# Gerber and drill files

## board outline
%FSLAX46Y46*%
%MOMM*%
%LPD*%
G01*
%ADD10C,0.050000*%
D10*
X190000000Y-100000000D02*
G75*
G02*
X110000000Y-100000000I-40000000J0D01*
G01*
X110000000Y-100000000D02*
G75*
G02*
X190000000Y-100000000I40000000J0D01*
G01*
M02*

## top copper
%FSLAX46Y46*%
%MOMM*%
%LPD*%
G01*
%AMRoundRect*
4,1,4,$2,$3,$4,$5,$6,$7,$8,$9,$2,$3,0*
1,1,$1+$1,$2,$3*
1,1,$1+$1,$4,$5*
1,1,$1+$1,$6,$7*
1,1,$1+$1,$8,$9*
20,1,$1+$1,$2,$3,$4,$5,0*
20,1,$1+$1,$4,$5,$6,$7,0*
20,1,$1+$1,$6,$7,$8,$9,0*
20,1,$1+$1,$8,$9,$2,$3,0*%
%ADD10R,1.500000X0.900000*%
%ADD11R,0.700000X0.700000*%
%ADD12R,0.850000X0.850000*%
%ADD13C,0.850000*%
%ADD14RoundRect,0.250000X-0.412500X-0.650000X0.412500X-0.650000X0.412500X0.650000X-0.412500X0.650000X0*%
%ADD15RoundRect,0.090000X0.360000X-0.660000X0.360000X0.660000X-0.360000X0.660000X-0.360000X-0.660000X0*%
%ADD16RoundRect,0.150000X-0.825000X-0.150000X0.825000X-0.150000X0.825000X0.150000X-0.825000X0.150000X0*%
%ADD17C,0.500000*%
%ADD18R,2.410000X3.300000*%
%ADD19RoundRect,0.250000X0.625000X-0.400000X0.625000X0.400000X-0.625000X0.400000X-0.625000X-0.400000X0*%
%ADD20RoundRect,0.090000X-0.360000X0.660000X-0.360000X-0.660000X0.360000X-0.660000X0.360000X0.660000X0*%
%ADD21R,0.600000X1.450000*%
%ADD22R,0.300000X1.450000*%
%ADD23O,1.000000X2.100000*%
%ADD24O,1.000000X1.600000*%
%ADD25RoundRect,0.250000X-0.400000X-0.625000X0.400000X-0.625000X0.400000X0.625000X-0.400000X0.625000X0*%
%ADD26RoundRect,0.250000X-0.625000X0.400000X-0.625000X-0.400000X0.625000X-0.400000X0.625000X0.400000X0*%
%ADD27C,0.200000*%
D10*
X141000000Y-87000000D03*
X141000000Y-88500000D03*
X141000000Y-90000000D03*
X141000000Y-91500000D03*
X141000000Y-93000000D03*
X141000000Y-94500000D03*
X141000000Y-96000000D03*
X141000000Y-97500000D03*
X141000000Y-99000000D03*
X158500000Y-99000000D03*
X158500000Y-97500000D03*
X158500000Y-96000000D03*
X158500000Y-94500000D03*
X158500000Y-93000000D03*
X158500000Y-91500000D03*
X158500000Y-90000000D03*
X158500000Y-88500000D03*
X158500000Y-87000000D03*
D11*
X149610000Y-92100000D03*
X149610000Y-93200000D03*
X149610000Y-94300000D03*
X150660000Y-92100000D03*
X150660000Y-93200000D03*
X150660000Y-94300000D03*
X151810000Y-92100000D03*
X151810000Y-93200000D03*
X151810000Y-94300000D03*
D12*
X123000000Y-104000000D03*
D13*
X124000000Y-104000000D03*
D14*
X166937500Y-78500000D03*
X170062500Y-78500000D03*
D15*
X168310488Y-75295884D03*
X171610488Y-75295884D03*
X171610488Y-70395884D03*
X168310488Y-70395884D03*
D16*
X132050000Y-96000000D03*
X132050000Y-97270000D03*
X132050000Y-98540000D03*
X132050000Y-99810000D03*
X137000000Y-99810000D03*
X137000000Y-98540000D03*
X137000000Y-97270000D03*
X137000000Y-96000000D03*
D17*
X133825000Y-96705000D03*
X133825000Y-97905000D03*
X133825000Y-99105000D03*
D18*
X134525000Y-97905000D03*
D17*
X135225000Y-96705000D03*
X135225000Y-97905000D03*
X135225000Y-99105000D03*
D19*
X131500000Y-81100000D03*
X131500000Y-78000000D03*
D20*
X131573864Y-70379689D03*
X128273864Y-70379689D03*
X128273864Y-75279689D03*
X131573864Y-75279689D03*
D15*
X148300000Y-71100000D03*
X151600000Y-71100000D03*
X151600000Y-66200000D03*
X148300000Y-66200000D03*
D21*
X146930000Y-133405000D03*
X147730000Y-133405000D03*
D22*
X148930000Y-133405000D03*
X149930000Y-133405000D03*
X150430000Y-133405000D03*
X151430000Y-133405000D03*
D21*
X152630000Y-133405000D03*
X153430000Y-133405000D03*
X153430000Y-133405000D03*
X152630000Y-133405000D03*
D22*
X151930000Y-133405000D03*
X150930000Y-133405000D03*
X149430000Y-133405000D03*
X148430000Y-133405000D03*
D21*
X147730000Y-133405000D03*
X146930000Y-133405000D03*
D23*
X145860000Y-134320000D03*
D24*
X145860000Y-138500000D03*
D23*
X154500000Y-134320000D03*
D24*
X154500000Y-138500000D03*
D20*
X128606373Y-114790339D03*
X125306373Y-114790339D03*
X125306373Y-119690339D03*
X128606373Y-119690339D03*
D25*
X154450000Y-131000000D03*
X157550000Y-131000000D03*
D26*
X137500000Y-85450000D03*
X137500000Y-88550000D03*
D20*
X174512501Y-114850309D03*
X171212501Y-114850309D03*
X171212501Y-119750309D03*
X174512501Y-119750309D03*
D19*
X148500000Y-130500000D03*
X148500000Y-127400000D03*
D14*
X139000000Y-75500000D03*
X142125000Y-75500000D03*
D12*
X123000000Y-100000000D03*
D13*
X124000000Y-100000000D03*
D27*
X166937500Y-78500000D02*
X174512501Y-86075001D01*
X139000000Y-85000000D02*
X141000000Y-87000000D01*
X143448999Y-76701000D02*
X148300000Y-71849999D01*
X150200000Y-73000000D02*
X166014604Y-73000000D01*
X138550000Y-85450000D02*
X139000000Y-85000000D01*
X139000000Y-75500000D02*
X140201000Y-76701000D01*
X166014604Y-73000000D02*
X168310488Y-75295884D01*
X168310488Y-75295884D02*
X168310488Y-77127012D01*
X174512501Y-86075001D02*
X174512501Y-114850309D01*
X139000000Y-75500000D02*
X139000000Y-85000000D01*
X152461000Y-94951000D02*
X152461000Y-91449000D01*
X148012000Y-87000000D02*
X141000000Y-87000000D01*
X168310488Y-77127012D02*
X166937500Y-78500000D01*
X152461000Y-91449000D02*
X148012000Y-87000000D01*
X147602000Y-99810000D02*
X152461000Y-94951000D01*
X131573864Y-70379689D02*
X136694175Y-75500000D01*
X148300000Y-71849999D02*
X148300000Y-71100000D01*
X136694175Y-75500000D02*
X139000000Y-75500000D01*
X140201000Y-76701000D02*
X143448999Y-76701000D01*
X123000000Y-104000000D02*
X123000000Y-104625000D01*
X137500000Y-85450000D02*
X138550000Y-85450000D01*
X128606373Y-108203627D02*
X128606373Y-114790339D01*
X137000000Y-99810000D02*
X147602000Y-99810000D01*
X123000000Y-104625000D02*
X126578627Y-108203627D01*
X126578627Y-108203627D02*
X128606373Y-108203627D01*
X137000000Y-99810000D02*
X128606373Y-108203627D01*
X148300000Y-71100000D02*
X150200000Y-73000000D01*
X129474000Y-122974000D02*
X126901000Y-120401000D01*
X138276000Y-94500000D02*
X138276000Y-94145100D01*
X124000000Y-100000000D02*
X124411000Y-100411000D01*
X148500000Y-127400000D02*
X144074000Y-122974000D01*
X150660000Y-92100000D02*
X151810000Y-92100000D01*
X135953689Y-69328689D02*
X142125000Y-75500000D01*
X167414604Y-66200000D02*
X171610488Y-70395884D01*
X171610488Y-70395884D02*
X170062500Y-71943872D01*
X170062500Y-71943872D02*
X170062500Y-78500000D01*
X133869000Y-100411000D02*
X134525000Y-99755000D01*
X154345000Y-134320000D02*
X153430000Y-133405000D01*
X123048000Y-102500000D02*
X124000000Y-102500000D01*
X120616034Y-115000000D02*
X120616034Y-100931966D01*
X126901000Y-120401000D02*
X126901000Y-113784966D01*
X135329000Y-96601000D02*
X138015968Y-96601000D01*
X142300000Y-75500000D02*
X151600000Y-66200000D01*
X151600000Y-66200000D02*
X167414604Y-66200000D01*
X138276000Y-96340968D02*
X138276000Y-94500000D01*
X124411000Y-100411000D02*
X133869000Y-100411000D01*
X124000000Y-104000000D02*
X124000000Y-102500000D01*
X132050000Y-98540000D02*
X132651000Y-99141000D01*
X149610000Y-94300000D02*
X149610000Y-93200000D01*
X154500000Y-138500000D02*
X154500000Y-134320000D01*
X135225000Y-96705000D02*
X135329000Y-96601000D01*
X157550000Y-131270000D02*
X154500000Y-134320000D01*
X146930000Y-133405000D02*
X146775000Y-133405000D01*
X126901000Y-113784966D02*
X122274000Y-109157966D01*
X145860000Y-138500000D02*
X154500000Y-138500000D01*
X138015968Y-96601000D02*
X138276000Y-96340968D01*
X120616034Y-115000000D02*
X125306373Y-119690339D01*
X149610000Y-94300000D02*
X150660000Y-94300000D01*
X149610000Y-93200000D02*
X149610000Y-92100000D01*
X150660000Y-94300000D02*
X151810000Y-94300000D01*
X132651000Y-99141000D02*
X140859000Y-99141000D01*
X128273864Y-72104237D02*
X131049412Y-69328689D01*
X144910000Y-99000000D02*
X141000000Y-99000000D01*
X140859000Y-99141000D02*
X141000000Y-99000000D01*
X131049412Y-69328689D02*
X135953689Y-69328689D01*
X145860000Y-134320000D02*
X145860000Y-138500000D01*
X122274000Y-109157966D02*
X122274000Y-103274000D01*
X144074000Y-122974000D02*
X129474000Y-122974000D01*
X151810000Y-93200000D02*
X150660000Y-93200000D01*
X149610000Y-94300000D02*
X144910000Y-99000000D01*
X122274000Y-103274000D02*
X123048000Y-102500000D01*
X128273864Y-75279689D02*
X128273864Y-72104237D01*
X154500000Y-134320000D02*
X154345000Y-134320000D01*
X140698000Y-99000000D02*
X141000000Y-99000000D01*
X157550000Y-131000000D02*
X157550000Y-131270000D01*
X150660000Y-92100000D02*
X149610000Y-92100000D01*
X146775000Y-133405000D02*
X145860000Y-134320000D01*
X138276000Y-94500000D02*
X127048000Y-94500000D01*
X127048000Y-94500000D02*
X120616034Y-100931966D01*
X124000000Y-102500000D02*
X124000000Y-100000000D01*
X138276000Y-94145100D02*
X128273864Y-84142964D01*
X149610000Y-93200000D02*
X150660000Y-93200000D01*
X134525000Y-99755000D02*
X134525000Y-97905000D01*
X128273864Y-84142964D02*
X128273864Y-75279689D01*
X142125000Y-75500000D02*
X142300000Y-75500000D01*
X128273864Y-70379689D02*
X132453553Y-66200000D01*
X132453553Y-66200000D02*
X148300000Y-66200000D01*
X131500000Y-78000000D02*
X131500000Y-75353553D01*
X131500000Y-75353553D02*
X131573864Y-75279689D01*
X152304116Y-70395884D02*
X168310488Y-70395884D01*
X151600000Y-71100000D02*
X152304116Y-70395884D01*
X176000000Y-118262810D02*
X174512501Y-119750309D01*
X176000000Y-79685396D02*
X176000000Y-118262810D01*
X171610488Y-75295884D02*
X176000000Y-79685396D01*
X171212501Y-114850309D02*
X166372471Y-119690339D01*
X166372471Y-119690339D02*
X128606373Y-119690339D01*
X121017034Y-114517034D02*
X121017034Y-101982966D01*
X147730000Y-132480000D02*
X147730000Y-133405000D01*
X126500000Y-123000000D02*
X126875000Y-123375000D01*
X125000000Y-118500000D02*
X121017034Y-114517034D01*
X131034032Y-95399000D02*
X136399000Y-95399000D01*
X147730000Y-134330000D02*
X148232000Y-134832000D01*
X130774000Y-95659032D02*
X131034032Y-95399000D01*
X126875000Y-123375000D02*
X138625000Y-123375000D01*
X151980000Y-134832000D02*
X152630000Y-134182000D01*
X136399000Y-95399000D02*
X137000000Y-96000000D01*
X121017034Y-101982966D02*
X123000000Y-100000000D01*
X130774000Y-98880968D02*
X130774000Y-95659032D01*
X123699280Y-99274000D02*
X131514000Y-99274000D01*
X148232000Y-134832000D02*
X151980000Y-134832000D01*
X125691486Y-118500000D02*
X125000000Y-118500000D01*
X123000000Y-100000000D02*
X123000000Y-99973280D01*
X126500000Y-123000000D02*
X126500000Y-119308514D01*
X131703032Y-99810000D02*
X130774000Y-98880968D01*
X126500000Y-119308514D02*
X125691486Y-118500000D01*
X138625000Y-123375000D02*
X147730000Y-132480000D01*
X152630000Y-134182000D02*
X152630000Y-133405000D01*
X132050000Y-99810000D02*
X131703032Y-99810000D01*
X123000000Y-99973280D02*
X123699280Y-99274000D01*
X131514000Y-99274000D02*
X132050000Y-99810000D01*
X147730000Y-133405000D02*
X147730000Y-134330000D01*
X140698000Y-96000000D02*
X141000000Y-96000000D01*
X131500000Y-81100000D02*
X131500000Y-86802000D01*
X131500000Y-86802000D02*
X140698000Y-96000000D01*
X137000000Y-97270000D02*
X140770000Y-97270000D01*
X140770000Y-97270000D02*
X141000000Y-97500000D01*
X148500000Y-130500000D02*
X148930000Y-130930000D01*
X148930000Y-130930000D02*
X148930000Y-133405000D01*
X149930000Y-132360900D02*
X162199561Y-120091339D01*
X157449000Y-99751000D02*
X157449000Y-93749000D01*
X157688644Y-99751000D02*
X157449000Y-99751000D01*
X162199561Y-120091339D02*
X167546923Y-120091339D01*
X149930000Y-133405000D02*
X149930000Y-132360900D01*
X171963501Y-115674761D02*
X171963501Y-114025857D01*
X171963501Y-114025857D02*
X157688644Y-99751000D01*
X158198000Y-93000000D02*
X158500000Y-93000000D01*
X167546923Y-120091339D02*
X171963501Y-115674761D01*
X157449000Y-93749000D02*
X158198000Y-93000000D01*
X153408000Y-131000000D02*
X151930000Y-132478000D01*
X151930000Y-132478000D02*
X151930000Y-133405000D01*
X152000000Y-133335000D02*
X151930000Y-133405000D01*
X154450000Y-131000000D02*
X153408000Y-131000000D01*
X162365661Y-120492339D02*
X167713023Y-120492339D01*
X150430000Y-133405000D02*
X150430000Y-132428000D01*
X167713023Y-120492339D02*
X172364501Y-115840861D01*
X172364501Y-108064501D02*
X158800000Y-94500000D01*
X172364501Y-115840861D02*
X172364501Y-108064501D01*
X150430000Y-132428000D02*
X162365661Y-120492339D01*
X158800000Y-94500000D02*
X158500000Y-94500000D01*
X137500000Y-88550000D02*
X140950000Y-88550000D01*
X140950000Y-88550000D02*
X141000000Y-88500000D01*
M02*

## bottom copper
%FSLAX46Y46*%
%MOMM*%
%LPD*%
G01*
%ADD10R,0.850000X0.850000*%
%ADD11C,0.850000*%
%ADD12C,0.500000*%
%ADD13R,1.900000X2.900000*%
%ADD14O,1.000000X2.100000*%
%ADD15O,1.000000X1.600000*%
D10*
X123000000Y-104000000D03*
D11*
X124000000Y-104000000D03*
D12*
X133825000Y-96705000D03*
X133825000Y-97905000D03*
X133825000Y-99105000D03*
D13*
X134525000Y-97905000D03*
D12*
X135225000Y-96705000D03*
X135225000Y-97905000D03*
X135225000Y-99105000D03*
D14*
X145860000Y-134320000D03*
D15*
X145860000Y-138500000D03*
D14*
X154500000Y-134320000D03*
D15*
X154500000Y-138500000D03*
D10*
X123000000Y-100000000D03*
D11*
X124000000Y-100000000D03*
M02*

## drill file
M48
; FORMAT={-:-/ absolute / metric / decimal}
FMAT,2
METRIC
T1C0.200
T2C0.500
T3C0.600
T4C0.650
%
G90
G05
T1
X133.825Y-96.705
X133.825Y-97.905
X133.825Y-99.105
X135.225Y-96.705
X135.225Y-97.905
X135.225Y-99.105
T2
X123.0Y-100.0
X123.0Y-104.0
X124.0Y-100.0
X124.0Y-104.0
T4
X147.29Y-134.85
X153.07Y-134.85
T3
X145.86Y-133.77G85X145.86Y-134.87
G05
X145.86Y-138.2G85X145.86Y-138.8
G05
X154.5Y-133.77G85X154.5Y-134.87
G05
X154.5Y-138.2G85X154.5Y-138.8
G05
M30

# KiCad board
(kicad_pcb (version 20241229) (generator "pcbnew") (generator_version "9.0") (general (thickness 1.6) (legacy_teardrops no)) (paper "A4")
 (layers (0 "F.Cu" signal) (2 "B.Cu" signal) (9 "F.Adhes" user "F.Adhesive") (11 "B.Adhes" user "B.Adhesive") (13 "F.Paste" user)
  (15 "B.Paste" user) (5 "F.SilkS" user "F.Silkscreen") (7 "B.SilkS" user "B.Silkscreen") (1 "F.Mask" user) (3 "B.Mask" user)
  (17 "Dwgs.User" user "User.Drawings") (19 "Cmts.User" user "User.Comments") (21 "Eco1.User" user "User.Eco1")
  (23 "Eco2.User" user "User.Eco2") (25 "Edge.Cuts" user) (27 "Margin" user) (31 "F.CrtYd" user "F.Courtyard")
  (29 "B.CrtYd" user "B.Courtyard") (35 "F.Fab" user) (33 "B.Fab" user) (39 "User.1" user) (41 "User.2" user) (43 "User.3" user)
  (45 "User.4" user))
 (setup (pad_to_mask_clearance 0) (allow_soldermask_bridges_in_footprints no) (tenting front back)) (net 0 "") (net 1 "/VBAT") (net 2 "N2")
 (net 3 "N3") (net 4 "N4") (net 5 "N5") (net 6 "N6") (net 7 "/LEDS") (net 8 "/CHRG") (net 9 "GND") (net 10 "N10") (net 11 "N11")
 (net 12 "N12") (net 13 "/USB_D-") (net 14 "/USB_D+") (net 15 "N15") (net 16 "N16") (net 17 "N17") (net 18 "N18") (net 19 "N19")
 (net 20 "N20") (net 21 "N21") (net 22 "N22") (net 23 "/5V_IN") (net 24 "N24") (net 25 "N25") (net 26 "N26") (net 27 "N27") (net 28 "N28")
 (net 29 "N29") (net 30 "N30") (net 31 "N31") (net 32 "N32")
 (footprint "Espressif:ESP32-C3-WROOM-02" (layer "F.Cu") (at 149.75 92.9)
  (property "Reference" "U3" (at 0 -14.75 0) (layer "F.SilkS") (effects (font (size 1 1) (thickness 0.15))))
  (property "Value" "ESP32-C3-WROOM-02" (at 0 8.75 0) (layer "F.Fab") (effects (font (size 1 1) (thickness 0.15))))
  (pad "1" smd rect (at -8.75 -5.9) (size 1.5 0.9) (layers "F.Cu" "F.Mask" "F.Paste") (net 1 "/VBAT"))
  (pad "2" smd rect (at -8.75 -4.4) (size 1.5 0.9) (layers "F.Cu" "F.Mask" "F.Paste") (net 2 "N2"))
  (pad "3" smd rect (at -8.75 -2.9) (size 1.5 0.9) (layers "F.Cu" "F.Mask" "F.Paste") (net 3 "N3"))
  (pad "4" smd rect (at -8.75 -1.4) (size 1.5 0.9) (layers "F.Cu" "F.Mask" "F.Paste") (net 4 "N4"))
  (pad "5" smd rect (at -8.75 0.1) (size 1.5 0.9) (layers "F.Cu" "F.Mask" "F.Paste") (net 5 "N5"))
  (pad "6" smd rect (at -8.75 1.6) (size 1.5 0.9) (layers "F.Cu" "F.Mask" "F.Paste") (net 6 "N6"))
  (pad "7" smd rect (at -8.75 3.1) (size 1.5 0.9) (layers "F.Cu" "F.Mask" "F.Paste") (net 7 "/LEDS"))
  (pad "8" smd rect (at -8.75 4.6) (size 1.5 0.9) (layers "F.Cu" "F.Mask" "F.Paste") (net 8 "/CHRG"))
  (pad "9" smd rect (at -8.75 6.1) (size 1.5 0.9) (layers "F.Cu" "F.Mask" "F.Paste") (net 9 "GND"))
  (pad "10" smd rect (at 8.75 6.1 180) (size 1.5 0.9) (layers "F.Cu" "F.Mask" "F.Paste") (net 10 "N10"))
  (pad "11" smd rect (at 8.75 4.6 180) (size 1.5 0.9) (layers "F.Cu" "F.Mask" "F.Paste") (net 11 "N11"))
  (pad "12" smd rect (at 8.75 3.1 180) (size 1.5 0.9) (layers "F.Cu" "F.Mask" "F.Paste") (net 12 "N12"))
  (pad "13" smd rect (at 8.75 1.6 180) (size 1.5 0.9) (layers "F.Cu" "F.Mask" "F.Paste") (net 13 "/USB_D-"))
  (pad "14" smd rect (at 8.75 0.1 180) (size 1.5 0.9) (layers "F.Cu" "F.Mask" "F.Paste") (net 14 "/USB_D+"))
  (pad "15" smd rect (at 8.75 -1.4 180) (size 1.5 0.9) (layers "F.Cu" "F.Mask" "F.Paste") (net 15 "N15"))
  (pad "16" smd rect (at 8.75 -2.9 180) (size 1.5 0.9) (layers "F.Cu" "F.Mask" "F.Paste") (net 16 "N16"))
  (pad "17" smd rect (at 8.75 -4.4 180) (size 1.5 0.9) (layers "F.Cu" "F.Mask" "F.Paste") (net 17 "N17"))
  (pad "18" smd rect (at 8.75 -5.9 180) (size 1.5 0.9) (layers "F.Cu" "F.Mask" "F.Paste") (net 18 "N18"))
  (pad "19" smd rect (at -0.14 -0.8 180) (size 0.7 0.7) (layers "F.Cu" "F.Mask" "F.Paste") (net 9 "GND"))
  (pad "19" smd rect (at -0.14 0.3 180) (size 0.7 0.7) (layers "F.Cu" "F.Mask" "F.Paste") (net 9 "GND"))
  (pad "19" smd rect (at -0.14 1.4 180) (size 0.7 0.7) (layers "F.Cu" "F.Mask" "F.Paste") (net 9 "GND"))
  (pad "19" smd rect (at 0.91 -0.8 180) (size 0.7 0.7) (layers "F.Cu" "F.Mask" "F.Paste") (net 9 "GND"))
  (pad "19" smd rect (at 0.91 0.3 180) (size 0.7 0.7) (layers "F.Cu" "F.Mask" "F.Paste") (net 9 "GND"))
  (pad "19" smd rect (at 0.91 1.4 180) (size 0.7 0.7) (layers "F.Cu" "F.Mask" "F.Paste") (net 9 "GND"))
  (pad "19" smd rect (at 2.06 -0.8 180) (size 0.7 0.7) (layers "F.Cu" "F.Mask" "F.Paste") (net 9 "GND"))
  (pad "19" smd rect (at 2.06 0.3 180) (size 0.7 0.7) (layers "F.Cu" "F.Mask" "F.Paste") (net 9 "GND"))
  (pad "19" smd rect (at 2.06 1.4 180) (size 0.7 0.7) (layers "F.Cu" "F.Mask" "F.Paste") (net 9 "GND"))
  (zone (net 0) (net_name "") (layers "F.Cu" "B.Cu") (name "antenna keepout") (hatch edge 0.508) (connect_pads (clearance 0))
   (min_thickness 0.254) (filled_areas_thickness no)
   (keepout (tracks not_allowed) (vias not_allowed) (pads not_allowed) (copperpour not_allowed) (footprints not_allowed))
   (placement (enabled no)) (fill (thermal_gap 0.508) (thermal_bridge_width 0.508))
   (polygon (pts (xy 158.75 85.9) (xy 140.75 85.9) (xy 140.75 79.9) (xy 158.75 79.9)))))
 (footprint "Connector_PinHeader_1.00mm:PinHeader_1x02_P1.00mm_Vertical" (layer "F.Cu") (at 123 104 90)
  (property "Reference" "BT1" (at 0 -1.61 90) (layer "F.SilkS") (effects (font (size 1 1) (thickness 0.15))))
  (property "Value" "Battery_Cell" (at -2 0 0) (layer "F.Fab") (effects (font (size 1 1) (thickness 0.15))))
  (pad "1" thru_hole rect (at 0 0 90) (size 0.85 0.85) (drill 0.5) (layers "*.Cu" "*.Mask") (remove_unused_layers no) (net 1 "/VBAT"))
  (pad "2" thru_hole circle (at 0 1 90) (size 0.85 0.85) (drill 0.5) (layers "*.Cu" "*.Mask") (remove_unused_layers no) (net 9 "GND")))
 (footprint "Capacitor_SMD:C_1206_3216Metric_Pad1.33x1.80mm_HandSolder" (layer "F.Cu") (at 168.5 78.5)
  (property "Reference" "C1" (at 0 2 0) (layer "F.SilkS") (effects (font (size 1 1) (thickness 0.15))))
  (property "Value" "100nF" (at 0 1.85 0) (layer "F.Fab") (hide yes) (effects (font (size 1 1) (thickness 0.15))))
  (pad "1" smd roundrect (at -1.5625 0) (size 1.325 1.8) (layers "F.Cu" "F.Mask" "F.Paste") (roundrect_rratio 0.188679) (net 1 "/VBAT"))
  (pad "2" smd roundrect (at 1.5625 0) (size 1.325 1.8) (layers "F.Cu" "F.Mask" "F.Paste") (roundrect_rratio 0.188679) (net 9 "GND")))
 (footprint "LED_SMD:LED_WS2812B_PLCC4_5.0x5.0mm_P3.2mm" (layer "F.Cu") (at 169.960488 72.845884 90)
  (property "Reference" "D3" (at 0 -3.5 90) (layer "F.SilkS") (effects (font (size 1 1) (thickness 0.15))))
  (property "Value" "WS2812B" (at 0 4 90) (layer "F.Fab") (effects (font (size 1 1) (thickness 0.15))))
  (pad "1" smd roundrect (at -2.45 -1.65 90) (size 1.5 0.9) (layers "F.Cu" "F.Mask" "F.Paste") (roundrect_rratio 0.1) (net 1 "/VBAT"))
  (pad "2" smd roundrect (at -2.45 1.65 90) (size 1.5 0.9) (layers "F.Cu" "F.Mask" "F.Paste") (roundrect_rratio 0.1) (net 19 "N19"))
  (pad "3" smd roundrect (at 2.45 1.65 90) (size 1.5 0.9) (layers "F.Cu" "F.Mask" "F.Paste") (roundrect_rratio 0.1) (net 9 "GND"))
  (pad "4" smd roundrect (at 2.45 -1.65 90) (size 1.5 0.9) (layers "F.Cu" "F.Mask" "F.Paste") (roundrect_rratio 0.1) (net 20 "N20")))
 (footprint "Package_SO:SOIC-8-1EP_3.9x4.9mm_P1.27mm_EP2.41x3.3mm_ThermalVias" (layer "F.Cu") (at 134.525 97.905)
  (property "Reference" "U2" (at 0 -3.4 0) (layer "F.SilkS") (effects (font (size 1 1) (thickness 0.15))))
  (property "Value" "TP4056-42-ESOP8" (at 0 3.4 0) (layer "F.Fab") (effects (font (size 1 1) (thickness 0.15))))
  (pad "" smd roundrect (at -0.6 -0.825) (size 1.01 1.38) (layers "F.Paste") (roundrect_rratio 0.247525))
  (pad "" smd roundrect (at -0.6 0.825) (size 1.01 1.38) (layers "F.Paste") (roundrect_rratio 0.247525))
  (pad "" smd roundrect (at 0.6 -0.825) (size 1.01 1.38) (layers "F.Paste") (roundrect_rratio 0.247525))
  (pad "" smd roundrect (at 0.6 0.825) (size 1.01 1.38) (layers "F.Paste") (roundrect_rratio 0.247525))
  (pad "1" smd roundrect (at -2.475 -1.905) (size 1.95 0.6) (layers "F.Cu" "F.Mask" "F.Paste") (roundrect_rratio 0.25) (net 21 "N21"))
  (pad "2" smd roundrect (at -2.475 -0.635) (size 1.95 0.6) (layers "F.Cu" "F.Mask" "F.Paste") (roundrect_rratio 0.25) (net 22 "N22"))
  (pad "3" smd roundrect (at -2.475 0.635) (size 1.95 0.6) (layers "F.Cu" "F.Mask" "F.Paste") (roundrect_rratio 0.25) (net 9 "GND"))
  (pad "4" smd roundrect (at -2.475 1.905) (size 1.95 0.6) (layers "F.Cu" "F.Mask" "F.Paste") (roundrect_rratio 0.25) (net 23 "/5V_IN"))
  (pad "5" smd roundrect (at 2.475 1.905) (size 1.95 0.6) (layers "F.Cu" "F.Mask" "F.Paste") (roundrect_rratio 0.25) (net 1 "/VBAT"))
  (pad "6" smd roundrect (at 2.475 0.635) (size 1.95 0.6) (layers "F.Cu" "F.Mask" "F.Paste") (roundrect_rratio 0.25) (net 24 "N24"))
  (pad "7" smd roundrect (at 2.475 -0.635) (size 1.95 0.6) (layers "F.Cu" "F.Mask" "F.Paste") (roundrect_rratio 0.25) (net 8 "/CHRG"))
  (pad "8" smd roundrect (at 2.475 -1.905) (size 1.95 0.6) (layers "F.Cu" "F.Mask" "F.Paste") (roundrect_rratio 0.25) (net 23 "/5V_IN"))
  (pad "9" thru_hole circle (at -0.7 -1.2) (size 0.5 0.5) (drill 0.2) (layers "*.Cu") (remove_unused_layers no) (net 9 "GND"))
  (pad "9" thru_hole circle (at -0.7 0) (size 0.5 0.5) (drill 0.2) (layers "*.Cu") (remove_unused_layers no) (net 9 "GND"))
  (pad "9" thru_hole circle (at -0.7 1.2) (size 0.5 0.5) (drill 0.2) (layers "*.Cu") (remove_unused_layers no) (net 9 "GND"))
  (pad "9" smd rect (at 0 0) (size 1.9 2.9) (layers "B.Cu") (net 9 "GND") (zone_connect 2))
  (pad "9" smd rect (at 0 0) (size 2.41 3.3) (layers "F.Cu" "F.Mask") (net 9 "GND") (zone_connect 2))
  (pad "9" thru_hole circle (at 0.7 -1.2) (size 0.5 0.5) (drill 0.2) (layers "*.Cu") (remove_unused_layers no) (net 9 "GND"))
  (pad "9" thru_hole circle (at 0.7 0) (size 0.5 0.5) (drill 0.2) (layers "*.Cu") (remove_unused_layers no) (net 9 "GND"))
  (pad "9" thru_hole circle (at 0.7 1.2) (size 0.5 0.5) (drill 0.2) (layers "*.Cu") (remove_unused_layers no) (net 9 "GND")))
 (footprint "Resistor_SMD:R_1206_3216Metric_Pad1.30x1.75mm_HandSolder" (layer "F.Cu") (at 131.5 79.55 90)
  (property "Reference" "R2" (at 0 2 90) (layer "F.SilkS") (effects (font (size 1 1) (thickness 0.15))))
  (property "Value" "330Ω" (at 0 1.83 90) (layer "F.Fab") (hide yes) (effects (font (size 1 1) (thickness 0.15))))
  (pad "1" smd roundrect (at -1.55 0 90) (size 1.3 1.75) (layers "F.Cu" "F.Mask" "F.Paste") (roundrect_rratio 0.192308) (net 7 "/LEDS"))
  (pad "2" smd roundrect (at 1.55 0 90) (size 1.3 1.75) (layers "F.Cu" "F.Mask" "F.Paste") (roundrect_rratio 0.192308) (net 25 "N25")))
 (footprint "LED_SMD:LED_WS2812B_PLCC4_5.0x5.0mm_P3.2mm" (layer "F.Cu") (at 129.923864 72.829689 -90)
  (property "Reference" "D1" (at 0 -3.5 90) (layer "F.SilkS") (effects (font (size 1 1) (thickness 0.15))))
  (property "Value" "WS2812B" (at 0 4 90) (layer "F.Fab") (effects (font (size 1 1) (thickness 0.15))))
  (pad "1" smd roundrect (at -2.45 -1.65 270) (size 1.5 0.9) (layers "F.Cu" "F.Mask" "F.Paste") (roundrect_rratio 0.1) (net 1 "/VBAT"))
  (pad "2" smd roundrect (at -2.45 1.65 270) (size 1.5 0.9) (layers "F.Cu" "F.Mask" "F.Paste") (roundrect_rratio 0.1) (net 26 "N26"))
  (pad "3" smd roundrect (at 2.45 1.65 270) (size 1.5 0.9) (layers "F.Cu" "F.Mask" "F.Paste") (roundrect_rratio 0.1) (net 9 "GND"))
  (pad "4" smd roundrect (at 2.45 -1.65 270) (size 1.5 0.9) (layers "F.Cu" "F.Mask" "F.Paste") (roundrect_rratio 0.1) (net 25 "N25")))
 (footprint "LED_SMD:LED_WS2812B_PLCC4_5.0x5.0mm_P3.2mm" (layer "F.Cu") (at 149.95 68.65 90)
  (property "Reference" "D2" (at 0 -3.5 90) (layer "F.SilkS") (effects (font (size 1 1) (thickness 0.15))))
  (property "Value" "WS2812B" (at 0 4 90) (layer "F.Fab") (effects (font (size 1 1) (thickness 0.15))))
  (pad "1" smd roundrect (at -2.45 -1.65 90) (size 1.5 0.9) (layers "F.Cu" "F.Mask" "F.Paste") (roundrect_rratio 0.1) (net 1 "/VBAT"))
  (pad "2" smd roundrect (at -2.45 1.65 90) (size 1.5 0.9) (layers "F.Cu" "F.Mask" "F.Paste") (roundrect_rratio 0.1) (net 20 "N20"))
  (pad "3" smd roundrect (at 2.45 1.65 90) (size 1.5 0.9) (layers "F.Cu" "F.Mask" "F.Paste") (roundrect_rratio 0.1) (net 9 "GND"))
  (pad "4" smd roundrect (at 2.45 -1.65 90) (size 1.5 0.9) (layers "F.Cu" "F.Mask" "F.Paste") (roundrect_rratio 0.1) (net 26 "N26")))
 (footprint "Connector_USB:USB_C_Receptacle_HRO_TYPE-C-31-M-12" (layer "F.Cu") (at 150.18 137.45)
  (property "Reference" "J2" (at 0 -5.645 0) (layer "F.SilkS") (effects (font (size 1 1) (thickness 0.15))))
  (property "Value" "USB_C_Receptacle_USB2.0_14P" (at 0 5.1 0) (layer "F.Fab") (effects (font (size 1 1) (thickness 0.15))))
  (pad "" np_thru_hole circle (at -2.89 -2.6) (size 0.65 0.65) (drill 0.65) (layers "*.Cu" "*.Mask"))
  (pad "" np_thru_hole circle (at 2.89 -2.6) (size 0.65 0.65) (drill 0.65) (layers "*.Cu" "*.Mask"))
  (pad "A1" smd rect (at -3.25 -4.045) (size 0.6 1.45) (layers "F.Cu" "F.Mask" "F.Paste") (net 9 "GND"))
  (pad "A4" smd rect (at -2.45 -4.045) (size 0.6 1.45) (layers "F.Cu" "F.Mask" "F.Paste") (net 23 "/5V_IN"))
  (pad "A5" smd rect (at -1.25 -4.045) (size 0.3 1.45) (layers "F.Cu" "F.Mask" "F.Paste") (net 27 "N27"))
  (pad "A6" smd rect (at -0.25 -4.045) (size 0.3 1.45) (layers "F.Cu" "F.Mask" "F.Paste") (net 14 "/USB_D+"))
  (pad "A7" smd rect (at 0.25 -4.045) (size 0.3 1.45) (layers "F.Cu" "F.Mask" "F.Paste") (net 13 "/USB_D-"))
  (pad "A8" smd rect (at 1.25 -4.045) (size 0.3 1.45) (layers "F.Cu" "F.Mask" "F.Paste"))
  (pad "A9" smd rect (at 2.45 -4.045) (size 0.6 1.45) (layers "F.Cu" "F.Mask" "F.Paste") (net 23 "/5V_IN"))
  (pad "A12" smd rect (at 3.25 -4.045) (size 0.6 1.45) (layers "F.Cu" "F.Mask" "F.Paste") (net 9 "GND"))
  (pad "B1" smd rect (at 3.25 -4.045) (size 0.6 1.45) (layers "F.Cu" "F.Mask" "F.Paste") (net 9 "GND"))
  (pad "B4" smd rect (at 2.45 -4.045) (size 0.6 1.45) (layers "F.Cu" "F.Mask" "F.Paste") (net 23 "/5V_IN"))
  (pad "B5" smd rect (at 1.75 -4.045) (size 0.3 1.45) (layers "F.Cu" "F.Mask" "F.Paste") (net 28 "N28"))
  (pad "B6" smd rect (at 0.75 -4.045) (size 0.3 1.45) (layers "F.Cu" "F.Mask" "F.Paste") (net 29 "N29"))
  (pad "B7" smd rect (at -0.75 -4.045) (size 0.3 1.45) (layers "F.Cu" "F.Mask" "F.Paste") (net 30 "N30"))
  (pad "B8" smd rect (at -1.75 -4.045) (size 0.3 1.45) (layers "F.Cu" "F.Mask" "F.Paste"))
  (pad "B9" smd rect (at -2.45 -4.045) (size 0.6 1.45) (layers "F.Cu" "F.Mask" "F.Paste") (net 23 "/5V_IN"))
  (pad "B12" smd rect (at -3.25 -4.045) (size 0.6 1.45) (layers "F.Cu" "F.Mask" "F.Paste") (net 9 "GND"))
  (pad "S1" thru_hole oval (at -4.32 -3.13) (size 1 2.1) (drill oval 0.6 1.7) (layers "*.Cu" "*.Mask") (remove_unused_layers no)
   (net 9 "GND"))
  (pad "S1" thru_hole oval (at -4.32 1.05) (size 1 1.6) (drill oval 0.6 1.2) (layers "*.Cu" "*.Mask") (remove_unused_layers no)
   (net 9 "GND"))
  (pad "S1" thru_hole oval (at 4.32 -3.13) (size 1 2.1) (drill oval 0.6 1.7) (layers "*.Cu" "*.Mask") (remove_unused_layers no)
   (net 9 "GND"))
  (pad "S1" thru_hole oval (at 4.32 1.05) (size 1 1.6) (drill oval 0.6 1.2) (layers "*.Cu" "*.Mask") (remove_unused_layers no) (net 9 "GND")))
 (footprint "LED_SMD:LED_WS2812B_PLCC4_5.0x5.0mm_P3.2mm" (layer "F.Cu") (at 126.956373 117.240339 -90)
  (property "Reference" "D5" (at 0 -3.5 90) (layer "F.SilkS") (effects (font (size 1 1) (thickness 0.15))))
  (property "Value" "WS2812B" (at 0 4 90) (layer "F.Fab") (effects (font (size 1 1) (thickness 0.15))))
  (pad "1" smd roundrect (at -2.45 -1.65 270) (size 1.5 0.9) (layers "F.Cu" "F.Mask" "F.Paste") (roundrect_rratio 0.1) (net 1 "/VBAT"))
  (pad "2" smd roundrect (at -2.45 1.65 270) (size 1.5 0.9) (layers "F.Cu" "F.Mask" "F.Paste") (roundrect_rratio 0.1) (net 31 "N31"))
  (pad "3" smd roundrect (at 2.45 1.65 270) (size 1.5 0.9) (layers "F.Cu" "F.Mask" "F.Paste") (roundrect_rratio 0.1) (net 9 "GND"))
  (pad "4" smd roundrect (at 2.45 -1.65 270) (size 1.5 0.9) (layers "F.Cu" "F.Mask" "F.Paste") (roundrect_rratio 0.1) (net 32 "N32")))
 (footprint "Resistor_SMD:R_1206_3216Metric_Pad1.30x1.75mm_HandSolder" (layer "F.Cu") (at 156 131)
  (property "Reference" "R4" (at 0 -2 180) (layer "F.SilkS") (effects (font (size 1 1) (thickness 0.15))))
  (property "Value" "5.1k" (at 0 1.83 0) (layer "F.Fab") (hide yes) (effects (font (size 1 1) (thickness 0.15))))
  (pad "1" smd roundrect (at -1.55 0) (size 1.3 1.75) (layers "F.Cu" "F.Mask" "F.Paste") (roundrect_rratio 0.192308) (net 28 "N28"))
  (pad "2" smd roundrect (at 1.55 0) (size 1.3 1.75) (layers "F.Cu" "F.Mask" "F.Paste") (roundrect_rratio 0.192308) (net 9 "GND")))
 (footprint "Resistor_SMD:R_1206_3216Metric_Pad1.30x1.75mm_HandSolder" (layer "F.Cu") (at 137.5 87 -90)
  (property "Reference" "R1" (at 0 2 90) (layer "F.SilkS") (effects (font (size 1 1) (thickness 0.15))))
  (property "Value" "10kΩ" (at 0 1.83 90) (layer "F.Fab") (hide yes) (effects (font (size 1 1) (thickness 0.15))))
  (pad "1" smd roundrect (at -1.55 0 270) (size 1.3 1.75) (layers "F.Cu" "F.Mask" "F.Paste") (roundrect_rratio 0.192308) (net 1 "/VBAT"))
  (pad "2" smd roundrect (at 1.55 0 270) (size 1.3 1.75) (layers "F.Cu" "F.Mask" "F.Paste") (roundrect_rratio 0.192308) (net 2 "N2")))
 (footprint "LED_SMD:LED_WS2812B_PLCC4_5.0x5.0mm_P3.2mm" (layer "F.Cu") (at 172.862501 117.300309 -90)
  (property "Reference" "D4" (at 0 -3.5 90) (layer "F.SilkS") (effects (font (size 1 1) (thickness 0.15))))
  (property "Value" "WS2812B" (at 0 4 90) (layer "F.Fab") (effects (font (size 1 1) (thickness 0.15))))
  (pad "1" smd roundrect (at -2.45 -1.65 270) (size 1.5 0.9) (layers "F.Cu" "F.Mask" "F.Paste") (roundrect_rratio 0.1) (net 1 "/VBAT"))
  (pad "2" smd roundrect (at -2.45 1.65 270) (size 1.5 0.9) (layers "F.Cu" "F.Mask" "F.Paste") (roundrect_rratio 0.1) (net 32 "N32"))
  (pad "3" smd roundrect (at 2.45 1.65 270) (size 1.5 0.9) (layers "F.Cu" "F.Mask" "F.Paste") (roundrect_rratio 0.1) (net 9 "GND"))
  (pad "4" smd roundrect (at 2.45 -1.65 270) (size 1.5 0.9) (layers "F.Cu" "F.Mask" "F.Paste") (roundrect_rratio 0.1) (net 19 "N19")))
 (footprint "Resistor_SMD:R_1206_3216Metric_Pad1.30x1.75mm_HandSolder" (layer "F.Cu") (at 148.5 128.95 90)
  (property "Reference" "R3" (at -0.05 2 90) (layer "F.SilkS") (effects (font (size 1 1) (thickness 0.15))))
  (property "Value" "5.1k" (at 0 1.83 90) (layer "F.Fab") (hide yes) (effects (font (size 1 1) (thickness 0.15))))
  (pad "1" smd roundrect (at -1.55 0 90) (size 1.3 1.75) (layers "F.Cu" "F.Mask" "F.Paste") (roundrect_rratio 0.192308) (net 27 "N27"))
  (pad "2" smd roundrect (at 1.55 0 90) (size 1.3 1.75) (layers "F.Cu" "F.Mask" "F.Paste") (roundrect_rratio 0.192308) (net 9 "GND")))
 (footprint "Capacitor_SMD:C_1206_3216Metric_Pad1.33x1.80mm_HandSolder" (layer "F.Cu") (at 140.5625 75.5)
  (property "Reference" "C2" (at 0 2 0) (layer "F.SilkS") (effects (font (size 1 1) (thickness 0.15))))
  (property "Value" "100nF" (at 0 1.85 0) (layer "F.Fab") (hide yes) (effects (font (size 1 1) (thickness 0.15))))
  (pad "1" smd roundrect (at -1.5625 0) (size 1.325 1.8) (layers "F.Cu" "F.Mask" "F.Paste") (roundrect_rratio 0.188679) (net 1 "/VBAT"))
  (pad "2" smd roundrect (at 1.5625 0) (size 1.325 1.8) (layers "F.Cu" "F.Mask" "F.Paste") (roundrect_rratio 0.188679) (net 9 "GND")))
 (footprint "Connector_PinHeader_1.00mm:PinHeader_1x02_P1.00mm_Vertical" (layer "F.Cu") (at 123 100 90)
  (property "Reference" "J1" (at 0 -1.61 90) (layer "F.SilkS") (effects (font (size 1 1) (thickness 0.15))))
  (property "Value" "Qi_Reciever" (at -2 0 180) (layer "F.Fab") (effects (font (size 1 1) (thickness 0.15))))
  (pad "1" thru_hole rect (at 0 0 90) (size 0.85 0.85) (drill 0.5) (layers "*.Cu" "*.Mask") (remove_unused_layers no) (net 23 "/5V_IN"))
  (pad "2" thru_hole circle (at 0 1 90) (size 0.85 0.85) (drill 0.5) (layers "*.Cu" "*.Mask") (remove_unused_layers no) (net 9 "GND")))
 (gr_circle (center 150 100) (end 190 100) (stroke (width 0.05) (type default)) (fill no) (layer "Edge.Cuts"))
 (segment (start 166.9375 78.5) (end 174.512501 86.075001) (width 0.2) (layer "F.Cu") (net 1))
 (segment (start 139 85) (end 141 87) (width 0.2) (layer "F.Cu") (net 1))
 (segment (start 143.448999 76.701) (end 148.3 71.849999) (width 0.2) (layer "F.Cu") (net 1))
 (segment (start 150.2 73) (end 166.014604 73) (width 0.2) (layer "F.Cu") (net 1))
 (segment (start 138.55 85.45) (end 139 85) (width 0.2) (layer "F.Cu") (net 1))
 (segment (start 139 75.5) (end 140.201 76.701) (width 0.2) (layer "F.Cu") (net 1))
 (segment (start 166.014604 73) (end 168.310488 75.295884) (width 0.2) (layer "F.Cu") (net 1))
 (segment (start 168.310488 75.295884) (end 168.310488 77.127012) (width 0.2) (layer "F.Cu") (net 1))
 (segment (start 174.512501 86.075001) (end 174.512501 114.850309) (width 0.2) (layer "F.Cu") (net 1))
 (segment (start 139 75.5) (end 139 85) (width 0.2) (layer "F.Cu") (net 1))
 (segment (start 152.461 94.951) (end 152.461 91.449) (width 0.2) (layer "F.Cu") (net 1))
 (segment (start 148.012 87) (end 141 87) (width 0.2) (layer "F.Cu") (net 1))
 (segment (start 168.310488 77.127012) (end 166.9375 78.5) (width 0.2) (layer "F.Cu") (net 1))
 (segment (start 152.461 91.449) (end 148.012 87) (width 0.2) (layer "F.Cu") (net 1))
 (segment (start 147.602 99.81) (end 152.461 94.951) (width 0.2) (layer "F.Cu") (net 1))
 (segment (start 131.573864 70.379689) (end 136.694175 75.5) (width 0.2) (layer "F.Cu") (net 1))
 (segment (start 148.3 71.849999) (end 148.3 71.1) (width 0.2) (layer "F.Cu") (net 1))
 (segment (start 136.694175 75.5) (end 139 75.5) (width 0.2) (layer "F.Cu") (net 1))
 (segment (start 140.201 76.701) (end 143.448999 76.701) (width 0.2) (layer "F.Cu") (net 1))
 (segment (start 123 104) (end 123 104.625) (width 0.2) (layer "F.Cu") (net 1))
 (segment (start 137.5 85.45) (end 138.55 85.45) (width 0.2) (layer "F.Cu") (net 1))
 (segment (start 128.606373 108.203627) (end 128.606373 114.790339) (width 0.2) (layer "F.Cu") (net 1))
 (segment (start 137 99.81) (end 147.602 99.81) (width 0.2) (layer "F.Cu") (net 1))
 (segment (start 123 104.625) (end 126.578627 108.203627) (width 0.2) (layer "F.Cu") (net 1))
 (segment (start 126.578627 108.203627) (end 128.606373 108.203627) (width 0.2) (layer "F.Cu") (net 1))
 (segment (start 137 99.81) (end 128.606373 108.203627) (width 0.2) (layer "F.Cu") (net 1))
 (segment (start 148.3 71.1) (end 150.2 73) (width 0.2) (layer "F.Cu") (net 1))
 (segment (start 129.474 122.974) (end 126.901 120.401) (width 0.2) (layer "F.Cu") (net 9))
 (segment (start 138.276 94.5) (end 138.276 94.1451) (width 0.2) (layer "F.Cu") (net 9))
 (segment (start 124 100) (end 124.411 100.411) (width 0.2) (layer "F.Cu") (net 9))
 (segment (start 148.5 127.4) (end 144.074 122.974) (width 0.2) (layer "F.Cu") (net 9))
 (segment (start 150.66 92.1) (end 151.81 92.1) (width 0.2) (layer "F.Cu") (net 9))
 (segment (start 135.953689 69.328689) (end 142.125 75.5) (width 0.2) (layer "F.Cu") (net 9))
 (segment (start 167.414604 66.2) (end 171.610488 70.395884) (width 0.2) (layer "F.Cu") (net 9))
 (segment (start 171.610488 70.395884) (end 170.0625 71.943872) (width 0.2) (layer "F.Cu") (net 9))
 (segment (start 170.0625 71.943872) (end 170.0625 78.5) (width 0.2) (layer "F.Cu") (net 9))
 (segment (start 133.869 100.411) (end 134.525 99.755) (width 0.2) (layer "F.Cu") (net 9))
 (segment (start 154.345 134.32) (end 153.43 133.405) (width 0.2) (layer "F.Cu") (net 9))
 (segment (start 123.048 102.5) (end 124 102.5) (width 0.2) (layer "F.Cu") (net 9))
 (segment (start 120.616034 115) (end 120.616034 100.931966) (width 0.2) (layer "F.Cu") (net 9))
 (segment (start 126.901 120.401) (end 126.901 113.784966) (width 0.2) (layer "F.Cu") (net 9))
 (segment (start 135.329 96.601) (end 138.015968 96.601) (width 0.2) (layer "F.Cu") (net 9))
 (segment (start 142.3 75.5) (end 151.6 66.2) (width 0.2) (layer "F.Cu") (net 9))
 (segment (start 151.6 66.2) (end 167.414604 66.2) (width 0.2) (layer "F.Cu") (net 9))
 (segment (start 138.276 96.340968) (end 138.276 94.5) (width 0.2) (layer "F.Cu") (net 9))
 (segment (start 124.411 100.411) (end 133.869 100.411) (width 0.2) (layer "F.Cu") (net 9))
 (segment (start 124 104) (end 124 102.5) (width 0.2) (layer "F.Cu") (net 9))
 (segment (start 132.05 98.54) (end 132.651 99.141) (width 0.2) (layer "F.Cu") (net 9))
 (segment (start 149.61 94.3) (end 149.61 93.2) (width 0.2) (layer "F.Cu") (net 9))
 (segment (start 154.5 138.5) (end 154.5 134.32) (width 0.2) (layer "F.Cu") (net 9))
 (segment (start 135.225 96.705) (end 135.329 96.601) (width 0.2) (layer "F.Cu") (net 9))
 (segment (start 157.55 131.27) (end 154.5 134.32) (width 0.2) (layer "F.Cu") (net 9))
 (segment (start 146.93 133.405) (end 146.775 133.405) (width 0.2) (layer "F.Cu") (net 9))
 (segment (start 126.901 113.784966) (end 122.274 109.157966) (width 0.2) (layer "F.Cu") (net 9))
 (segment (start 145.86 138.5) (end 154.5 138.5) (width 0.2) (layer "F.Cu") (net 9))
 (segment (start 138.015968 96.601) (end 138.276 96.340968) (width 0.2) (layer "F.Cu") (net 9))
 (segment (start 120.616034 115) (end 125.306373 119.690339) (width 0.2) (layer "F.Cu") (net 9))
 (segment (start 149.61 94.3) (end 150.66 94.3) (width 0.2) (layer "F.Cu") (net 9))
 (segment (start 149.61 93.2) (end 149.61 92.1) (width 0.2) (layer "F.Cu") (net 9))
 (segment (start 150.66 94.3) (end 151.81 94.3) (width 0.2) (layer "F.Cu") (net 9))
 (segment (start 132.651 99.141) (end 140.859 99.141) (width 0.2) (layer "F.Cu") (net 9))
 (segment (start 128.273864 72.104237) (end 131.049412 69.328689) (width 0.2) (layer "F.Cu") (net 9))
 (segment (start 144.91 99) (end 141 99) (width 0.2) (layer "F.Cu") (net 9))
 (segment (start 140.859 99.141) (end 141 99) (width 0.2) (layer "F.Cu") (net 9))
 (segment (start 131.049412 69.328689) (end 135.953689 69.328689) (width 0.2) (layer "F.Cu") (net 9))
 (segment (start 145.86 134.32) (end 145.86 138.5) (width 0.2) (layer "F.Cu") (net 9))
 (segment (start 122.274 109.157966) (end 122.274 103.274) (width 0.2) (layer "F.Cu") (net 9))
 (segment (start 144.074 122.974) (end 129.474 122.974) (width 0.2) (layer "F.Cu") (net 9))
 (segment (start 151.81 93.2) (end 150.66 93.2) (width 0.2) (layer "F.Cu") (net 9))
 (segment (start 149.61 94.3) (end 144.91 99) (width 0.2) (layer "F.Cu") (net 9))
 (segment (start 122.274 103.274) (end 123.048 102.5) (width 0.2) (layer "F.Cu") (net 9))
 (segment (start 128.273864 75.279689) (end 128.273864 72.104237) (width 0.2) (layer "F.Cu") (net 9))
 (segment (start 154.5 134.32) (end 154.345 134.32) (width 0.2) (layer "F.Cu") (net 9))
 (segment (start 140.698 99) (end 141 99) (width 0.2) (layer "F.Cu") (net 9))
 (segment (start 157.55 131) (end 157.55 131.27) (width 0.2) (layer "F.Cu") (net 9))
 (segment (start 150.66 92.1) (end 149.61 92.1) (width 0.2) (layer "F.Cu") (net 9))
 (segment (start 146.775 133.405) (end 145.86 134.32) (width 0.2) (layer "F.Cu") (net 9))
 (segment (start 138.276 94.5) (end 127.048 94.5) (width 0.2) (layer "F.Cu") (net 9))
 (segment (start 127.048 94.5) (end 120.616034 100.931966) (width 0.2) (layer "F.Cu") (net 9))
 (segment (start 124 102.5) (end 124 100) (width 0.2) (layer "F.Cu") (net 9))
 (segment (start 138.276 94.1451) (end 128.273864 84.142964) (width 0.2) (layer "F.Cu") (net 9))
 (segment (start 149.61 93.2) (end 150.66 93.2) (width 0.2) (layer "F.Cu") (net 9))
 (segment (start 134.525 99.755) (end 134.525 97.905) (width 0.2) (layer "F.Cu") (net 9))
 (segment (start 128.273864 84.142964) (end 128.273864 75.279689) (width 0.2) (layer "F.Cu") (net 9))
 (segment (start 142.125 75.5) (end 142.3 75.5) (width 0.2) (layer "F.Cu") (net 9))
 (segment (start 128.273864 70.379689) (end 132.453553 66.2) (width 0.2) (layer "F.Cu") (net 26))
 (segment (start 132.453553 66.2) (end 148.3 66.2) (width 0.2) (layer "F.Cu") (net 26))
 (segment (start 131.5 78) (end 131.5 75.353553) (width 0.2) (layer "F.Cu") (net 25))
 (segment (start 131.5 75.353553) (end 131.573864 75.279689) (width 0.2) (layer "F.Cu") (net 25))
 (segment (start 152.304116 70.395884) (end 168.310488 70.395884) (width 0.2) (layer "F.Cu") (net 20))
 (segment (start 151.6 71.1) (end 152.304116 70.395884) (width 0.2) (layer "F.Cu") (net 20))
 (segment (start 176 118.26281) (end 174.512501 119.750309) (width 0.2) (layer "F.Cu") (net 19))
 (segment (start 176 79.685396) (end 176 118.26281) (width 0.2) (layer "F.Cu") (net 19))
 (segment (start 171.610488 75.295884) (end 176 79.685396) (width 0.2) (layer "F.Cu") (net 19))
 (segment (start 171.212501 114.850309) (end 166.372471 119.690339) (width 0.2) (layer "F.Cu") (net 32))
 (segment (start 166.372471 119.690339) (end 128.606373 119.690339) (width 0.2) (layer "F.Cu") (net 32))
 (segment (start 121.017034 114.517034) (end 121.017034 101.982966) (width 0.2) (layer "F.Cu") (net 23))
 (segment (start 147.73 132.48) (end 147.73 133.405) (width 0.2) (layer "F.Cu") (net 23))
 (segment (start 126.5 123) (end 126.875 123.375) (width 0.2) (layer "F.Cu") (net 23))
 (segment (start 125 118.5) (end 121.017034 114.517034) (width 0.2) (layer "F.Cu") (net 23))
 (segment (start 131.034032 95.399) (end 136.399 95.399) (width 0.2) (layer "F.Cu") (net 23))
 (segment (start 147.73 134.33) (end 148.232 134.832) (width 0.2) (layer "F.Cu") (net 23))
 (segment (start 130.774 95.659032) (end 131.034032 95.399) (width 0.2) (layer "F.Cu") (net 23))
 (segment (start 126.875 123.375) (end 138.625 123.375) (width 0.2) (layer "F.Cu") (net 23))
 (segment (start 151.98 134.832) (end 152.63 134.182) (width 0.2) (layer "F.Cu") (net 23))
 (segment (start 136.399 95.399) (end 137 96) (width 0.2) (layer "F.Cu") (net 23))
 (segment (start 121.017034 101.982966) (end 123 100) (width 0.2) (layer "F.Cu") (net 23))
 (segment (start 130.774 98.880968) (end 130.774 95.659032) (width 0.2) (layer "F.Cu") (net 23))
 (segment (start 123.69928 99.274) (end 131.514 99.274) (width 0.2) (layer "F.Cu") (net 23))
 (segment (start 148.232 134.832) (end 151.98 134.832) (width 0.2) (layer "F.Cu") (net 23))
 (segment (start 125.691486 118.5) (end 125 118.5) (width 0.2) (layer "F.Cu") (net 23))
 (segment (start 123 100) (end 123 99.97328) (width 0.2) (layer "F.Cu") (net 23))
 (segment (start 126.5 123) (end 126.5 119.308514) (width 0.2) (layer "F.Cu") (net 23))
 (segment (start 131.703032 99.81) (end 130.774 98.880968) (width 0.2) (layer "F.Cu") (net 23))
 (segment (start 126.5 119.308514) (end 125.691486 118.5) (width 0.2) (layer "F.Cu") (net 23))
 (segment (start 138.625 123.375) (end 147.73 132.48) (width 0.2) (layer "F.Cu") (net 23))
 (segment (start 152.63 134.182) (end 152.63 133.405) (width 0.2) (layer "F.Cu") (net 23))
 (segment (start 132.05 99.81) (end 131.703032 99.81) (width 0.2) (layer "F.Cu") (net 23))
 (segment (start 123 99.97328) (end 123.69928 99.274) (width 0.2) (layer "F.Cu") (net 23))
 (segment (start 131.514 99.274) (end 132.05 99.81) (width 0.2) (layer "F.Cu") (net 23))
 (segment (start 147.73 133.405) (end 147.73 134.33) (width 0.2) (layer "F.Cu") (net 23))
 (segment (start 140.698 96) (end 141 96) (width 0.2) (layer "F.Cu") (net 7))
 (segment (start 131.5 81.1) (end 131.5 86.802) (width 0.2) (layer "F.Cu") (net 7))
 (segment (start 131.5 86.802) (end 140.698 96) (width 0.2) (layer "F.Cu") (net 7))
 (segment (start 137 97.27) (end 140.77 97.27) (width 0.2) (layer "F.Cu") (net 8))
 (segment (start 140.77 97.27) (end 141 97.5) (width 0.2) (layer "F.Cu") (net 8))
 (segment (start 148.5 130.5) (end 148.93 130.93) (width 0.2) (layer "F.Cu") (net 27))
 (segment (start 148.93 130.93) (end 148.93 133.405) (width 0.2) (layer "F.Cu") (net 27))
 (segment (start 149.93 132.3609) (end 162.199561 120.091339) (width 0.2) (layer "F.Cu") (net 14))
 (segment (start 157.449 99.751) (end 157.449 93.749) (width 0.2) (layer "F.Cu") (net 14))
 (segment (start 157.688644 99.751) (end 157.449 99.751) (width 0.2) (layer "F.Cu") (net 14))
 (segment (start 162.199561 120.091339) (end 167.546923 120.091339) (width 0.2) (layer "F.Cu") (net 14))
 (segment (start 149.93 133.405) (end 149.93 132.3609) (width 0.2) (layer "F.Cu") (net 14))
 (segment (start 171.963501 115.674761) (end 171.963501 114.025857) (width 0.2) (layer "F.Cu") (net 14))
 (segment (start 171.963501 114.025857) (end 157.688644 99.751) (width 0.2) (layer "F.Cu") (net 14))
 (segment (start 158.198 93) (end 158.5 93) (width 0.2) (layer "F.Cu") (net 14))
 (segment (start 167.546923 120.091339) (end 171.963501 115.674761) (width 0.2) (layer "F.Cu") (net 14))
 (segment (start 157.449 93.749) (end 158.198 93) (width 0.2) (layer "F.Cu") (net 14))
 (segment (start 153.408 131) (end 151.93 132.478) (width 0.2) (layer "F.Cu") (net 28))
 (segment (start 151.93 132.478) (end 151.93 133.405) (width 0.2) (layer "F.Cu") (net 28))
 (segment (start 152 133.335) (end 151.93 133.405) (width 0.2) (layer "F.Cu") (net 28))
 (segment (start 154.45 131) (end 153.408 131) (width 0.2) (layer "F.Cu") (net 28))
 (segment (start 162.365661 120.492339) (end 167.713023 120.492339) (width 0.2) (layer "F.Cu") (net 13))
 (segment (start 150.43 133.405) (end 150.43 132.428) (width 0.2) (layer "F.Cu") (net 13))
 (segment (start 167.713023 120.492339) (end 172.364501 115.840861) (width 0.2) (layer "F.Cu") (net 13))
 (segment (start 172.364501 108.064501) (end 158.8 94.5) (width 0.2) (layer "F.Cu") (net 13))
 (segment (start 172.364501 115.840861) (end 172.364501 108.064501) (width 0.2) (layer "F.Cu") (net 13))
 (segment (start 150.43 132.428) (end 162.365661 120.492339) (width 0.2) (layer "F.Cu") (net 13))
 (segment (start 158.8 94.5) (end 158.5 94.5) (width 0.2) (layer "F.Cu") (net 13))
 (segment (start 137.5 88.55) (end 140.95 88.55) (width 0.2) (layer "F.Cu") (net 2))
 (segment (start 140.95 88.55) (end 141 88.5) (width 0.2) (layer "F.Cu") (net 2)))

